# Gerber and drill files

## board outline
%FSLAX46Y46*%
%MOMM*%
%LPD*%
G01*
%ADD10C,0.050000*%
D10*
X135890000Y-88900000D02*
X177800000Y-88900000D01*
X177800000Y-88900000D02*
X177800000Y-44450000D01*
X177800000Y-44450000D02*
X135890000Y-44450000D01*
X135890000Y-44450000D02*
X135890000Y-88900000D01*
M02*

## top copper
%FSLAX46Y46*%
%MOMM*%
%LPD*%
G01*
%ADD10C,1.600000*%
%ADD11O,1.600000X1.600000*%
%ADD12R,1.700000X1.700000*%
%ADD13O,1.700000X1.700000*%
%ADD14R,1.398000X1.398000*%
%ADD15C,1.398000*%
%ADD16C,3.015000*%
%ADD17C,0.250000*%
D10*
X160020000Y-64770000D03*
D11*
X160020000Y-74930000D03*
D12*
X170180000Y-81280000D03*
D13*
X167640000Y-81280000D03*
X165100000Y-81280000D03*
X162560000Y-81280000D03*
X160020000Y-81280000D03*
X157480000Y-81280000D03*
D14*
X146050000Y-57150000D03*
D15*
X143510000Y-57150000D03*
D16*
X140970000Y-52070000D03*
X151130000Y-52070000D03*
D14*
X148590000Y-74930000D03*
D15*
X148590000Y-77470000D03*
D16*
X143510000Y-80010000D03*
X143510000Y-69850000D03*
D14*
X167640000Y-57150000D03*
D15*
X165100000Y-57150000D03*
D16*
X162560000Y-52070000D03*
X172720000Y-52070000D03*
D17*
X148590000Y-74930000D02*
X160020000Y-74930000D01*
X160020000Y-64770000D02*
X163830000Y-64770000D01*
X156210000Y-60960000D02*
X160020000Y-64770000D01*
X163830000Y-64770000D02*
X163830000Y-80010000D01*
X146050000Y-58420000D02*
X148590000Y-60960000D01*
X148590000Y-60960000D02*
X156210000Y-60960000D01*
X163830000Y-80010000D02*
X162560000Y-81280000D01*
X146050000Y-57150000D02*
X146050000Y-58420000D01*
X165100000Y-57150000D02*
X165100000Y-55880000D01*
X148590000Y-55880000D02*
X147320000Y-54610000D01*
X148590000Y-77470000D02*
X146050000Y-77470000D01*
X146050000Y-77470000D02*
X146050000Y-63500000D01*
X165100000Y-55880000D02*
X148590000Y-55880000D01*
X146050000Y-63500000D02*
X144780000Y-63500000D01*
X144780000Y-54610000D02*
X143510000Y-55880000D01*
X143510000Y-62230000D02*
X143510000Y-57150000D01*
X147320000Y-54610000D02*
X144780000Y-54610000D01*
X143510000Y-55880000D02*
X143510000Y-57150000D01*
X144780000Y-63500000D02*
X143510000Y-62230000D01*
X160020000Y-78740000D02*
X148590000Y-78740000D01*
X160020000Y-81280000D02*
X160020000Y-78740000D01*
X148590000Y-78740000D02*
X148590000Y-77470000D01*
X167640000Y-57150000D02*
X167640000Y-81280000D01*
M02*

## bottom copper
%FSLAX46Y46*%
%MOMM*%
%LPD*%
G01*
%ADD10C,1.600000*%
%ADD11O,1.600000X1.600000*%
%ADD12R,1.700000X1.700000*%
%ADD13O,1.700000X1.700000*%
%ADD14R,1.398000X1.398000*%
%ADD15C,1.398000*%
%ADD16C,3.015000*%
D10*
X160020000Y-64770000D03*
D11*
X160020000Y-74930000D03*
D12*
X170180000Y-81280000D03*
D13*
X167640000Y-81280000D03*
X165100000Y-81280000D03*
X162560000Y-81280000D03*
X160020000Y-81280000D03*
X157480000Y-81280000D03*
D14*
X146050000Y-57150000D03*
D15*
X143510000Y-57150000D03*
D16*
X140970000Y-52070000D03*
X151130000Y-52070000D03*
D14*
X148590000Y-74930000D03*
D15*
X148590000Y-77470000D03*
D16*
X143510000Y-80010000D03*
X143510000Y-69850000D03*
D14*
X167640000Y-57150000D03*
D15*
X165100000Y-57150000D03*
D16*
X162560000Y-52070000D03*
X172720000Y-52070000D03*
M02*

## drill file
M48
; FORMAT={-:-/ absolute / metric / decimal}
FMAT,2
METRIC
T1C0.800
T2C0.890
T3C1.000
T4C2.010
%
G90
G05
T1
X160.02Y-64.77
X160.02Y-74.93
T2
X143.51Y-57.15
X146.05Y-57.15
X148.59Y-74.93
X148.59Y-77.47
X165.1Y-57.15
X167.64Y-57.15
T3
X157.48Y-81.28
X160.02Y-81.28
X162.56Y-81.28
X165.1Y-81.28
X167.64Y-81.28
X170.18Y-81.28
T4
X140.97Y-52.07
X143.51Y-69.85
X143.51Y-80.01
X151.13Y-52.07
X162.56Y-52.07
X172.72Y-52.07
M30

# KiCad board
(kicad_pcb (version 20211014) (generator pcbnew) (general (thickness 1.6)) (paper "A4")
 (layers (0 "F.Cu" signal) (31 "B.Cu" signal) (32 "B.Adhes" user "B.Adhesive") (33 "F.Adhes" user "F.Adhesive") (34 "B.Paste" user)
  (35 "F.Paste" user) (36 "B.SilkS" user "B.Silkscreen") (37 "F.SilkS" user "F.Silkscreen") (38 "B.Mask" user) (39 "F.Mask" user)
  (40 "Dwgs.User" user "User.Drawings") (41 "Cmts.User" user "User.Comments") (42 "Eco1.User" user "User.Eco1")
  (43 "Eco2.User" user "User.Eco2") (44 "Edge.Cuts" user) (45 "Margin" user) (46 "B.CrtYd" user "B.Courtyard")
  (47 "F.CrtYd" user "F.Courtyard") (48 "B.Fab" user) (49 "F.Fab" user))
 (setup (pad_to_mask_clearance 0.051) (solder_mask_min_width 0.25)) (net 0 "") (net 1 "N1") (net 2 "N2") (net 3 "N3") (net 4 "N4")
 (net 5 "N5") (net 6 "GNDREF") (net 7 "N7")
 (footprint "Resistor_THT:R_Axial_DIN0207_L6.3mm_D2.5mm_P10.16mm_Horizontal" (layer "F.Cu") (at 160.02 64.77 -90)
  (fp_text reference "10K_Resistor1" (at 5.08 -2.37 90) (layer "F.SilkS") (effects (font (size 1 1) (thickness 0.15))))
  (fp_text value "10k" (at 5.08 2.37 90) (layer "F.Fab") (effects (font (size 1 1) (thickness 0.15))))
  (pad "1" thru_hole circle locked (at 0 0 270) (size 1.6 1.6) (drill 0.8) (layers *.Cu *.Mask) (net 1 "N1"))
  (pad "2" thru_hole oval locked (at 10.16 0 270) (size 1.6 1.6) (drill 0.8) (layers *.Cu *.Mask) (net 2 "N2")))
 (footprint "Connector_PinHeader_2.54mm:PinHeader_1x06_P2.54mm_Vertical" (layer "F.Cu") (at 170.18 81.28 -90)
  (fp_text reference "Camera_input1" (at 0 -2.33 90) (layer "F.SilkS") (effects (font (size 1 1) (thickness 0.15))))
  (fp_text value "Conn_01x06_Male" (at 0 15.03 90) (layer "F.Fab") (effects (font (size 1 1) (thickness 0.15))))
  (pad "1" thru_hole rect locked (at 0 0 270) (size 1.7 1.7) (drill 1) (layers *.Cu *.Mask) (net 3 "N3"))
  (pad "2" thru_hole oval locked (at 0 2.54 270) (size 1.7 1.7) (drill 1) (layers *.Cu *.Mask) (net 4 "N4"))
  (pad "3" thru_hole oval locked (at 0 5.08 270) (size 1.7 1.7) (drill 1) (layers *.Cu *.Mask) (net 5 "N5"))
  (pad "4" thru_hole oval locked (at 0 7.62 270) (size 1.7 1.7) (drill 1) (layers *.Cu *.Mask) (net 1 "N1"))
  (pad "5" thru_hole oval locked (at 0 10.16 270) (size 1.7 1.7) (drill 1) (layers *.Cu *.Mask) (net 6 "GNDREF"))
  (pad "6" thru_hole oval locked (at 0 12.7 270) (size 1.7 1.7) (drill 1) (layers *.Cu *.Mask) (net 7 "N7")))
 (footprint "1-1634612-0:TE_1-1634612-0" (layer "F.Cu") (at 146.05 57.15 90)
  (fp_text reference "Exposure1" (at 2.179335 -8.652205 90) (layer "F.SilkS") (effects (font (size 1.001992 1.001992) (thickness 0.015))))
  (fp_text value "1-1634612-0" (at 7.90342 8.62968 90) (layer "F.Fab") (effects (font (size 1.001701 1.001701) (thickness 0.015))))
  (pad "1" thru_hole rect locked (at 0 0 90) (size 1.398 1.398) (drill 0.89) (layers *.Cu *.Mask) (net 1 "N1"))
  (pad "2" thru_hole circle locked (at 0 -2.54 90) (size 1.398 1.398) (drill 0.89) (layers *.Cu *.Mask) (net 6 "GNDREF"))
  (pad "S1" thru_hole circle locked (at 5.08 -5.08 90) (size 3.015 3.015) (drill 2.01) (layers *.Cu *.Mask))
  (pad "S2" thru_hole circle locked (at 5.08 5.08 90) (size 3.015 3.015) (drill 2.01) (layers *.Cu *.Mask)))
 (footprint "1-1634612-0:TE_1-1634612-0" (layer "F.Cu") (at 148.59 74.93 180)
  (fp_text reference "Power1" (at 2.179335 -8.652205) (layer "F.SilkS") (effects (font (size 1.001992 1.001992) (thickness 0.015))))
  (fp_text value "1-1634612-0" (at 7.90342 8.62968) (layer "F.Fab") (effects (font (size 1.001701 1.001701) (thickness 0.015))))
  (pad "1" thru_hole rect locked (at 0 0 180) (size 1.398 1.398) (drill 0.89) (layers *.Cu *.Mask) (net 2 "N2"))
  (pad "2" thru_hole circle locked (at 0 -2.54 180) (size 1.398 1.398) (drill 0.89) (layers *.Cu *.Mask) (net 6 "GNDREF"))
  (pad "S1" thru_hole circle locked (at 5.08 -5.08 180) (size 3.015 3.015) (drill 2.01) (layers *.Cu *.Mask))
  (pad "S2" thru_hole circle locked (at 5.08 5.08 180) (size 3.015 3.015) (drill 2.01) (layers *.Cu *.Mask)))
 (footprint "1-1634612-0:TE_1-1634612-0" (layer "F.Cu") (at 167.64 57.15 90)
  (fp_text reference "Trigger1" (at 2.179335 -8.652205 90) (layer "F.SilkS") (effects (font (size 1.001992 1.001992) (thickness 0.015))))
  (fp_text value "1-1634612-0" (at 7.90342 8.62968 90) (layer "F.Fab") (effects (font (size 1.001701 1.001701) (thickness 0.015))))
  (pad "1" thru_hole rect locked (at 0 0 90) (size 1.398 1.398) (drill 0.89) (layers *.Cu *.Mask) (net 4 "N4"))
  (pad "2" thru_hole circle locked (at 0 -2.54 90) (size 1.398 1.398) (drill 0.89) (layers *.Cu *.Mask) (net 6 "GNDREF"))
  (pad "S1" thru_hole circle locked (at 5.08 -5.08 90) (size 3.015 3.015) (drill 2.01) (layers *.Cu *.Mask))
  (pad "S2" thru_hole circle locked (at 5.08 5.08 90) (size 3.015 3.015) (drill 2.01) (layers *.Cu *.Mask)))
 (gr_line (start 135.89 88.9) (end 177.8 88.9) (layer "Edge.Cuts") (width 0.05))
 (gr_line (start 177.8 88.9) (end 177.8 44.45) (layer "Edge.Cuts") (width 0.05))
 (gr_line (start 177.8 44.45) (end 135.89 44.45) (layer "Edge.Cuts") (width 0.05))
 (gr_line (start 135.89 44.45) (end 135.89 88.9) (layer "Edge.Cuts") (width 0.05))
 (segment (start 148.59 74.93) (end 160.02 74.93) (width 0.25) (layer "F.Cu") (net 2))
 (segment (start 160.02 64.77) (end 163.83 64.77) (width 0.25) (layer "F.Cu") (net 1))
 (segment (start 156.21 60.96) (end 160.02 64.77) (width 0.25) (layer "F.Cu") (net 1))
 (segment (start 163.83 64.77) (end 163.83 80.01) (width 0.25) (layer "F.Cu") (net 1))
 (segment (start 146.05 58.42) (end 148.59 60.96) (width 0.25) (layer "F.Cu") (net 1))
 (segment (start 148.59 60.96) (end 156.21 60.96) (width 0.25) (layer "F.Cu") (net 1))
 (segment (start 163.83 80.01) (end 162.56 81.28) (width 0.25) (layer "F.Cu") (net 1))
 (segment (start 146.05 57.15) (end 146.05 58.42) (width 0.25) (layer "F.Cu") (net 1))
 (segment (start 165.1 57.15) (end 165.1 55.88) (width 0.25) (layer "F.Cu") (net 6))
 (segment (start 148.59 55.88) (end 147.32 54.61) (width 0.25) (layer "F.Cu") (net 6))
 (segment (start 148.59 77.47) (end 146.05 77.47) (width 0.25) (layer "F.Cu") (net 6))
 (segment (start 146.05 77.47) (end 146.05 63.5) (width 0.25) (layer "F.Cu") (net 6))
 (segment (start 165.1 55.88) (end 148.59 55.88) (width 0.25) (layer "F.Cu") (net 6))
 (segment (start 146.05 63.5) (end 144.78 63.5) (width 0.25) (layer "F.Cu") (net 6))
 (segment (start 144.78 54.61) (end 143.51 55.88) (width 0.25) (layer "F.Cu") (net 6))
 (segment (start 143.51 62.23) (end 143.51 57.15) (width 0.25) (layer "F.Cu") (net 6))
 (segment (start 147.32 54.61) (end 144.78 54.61) (width 0.25) (layer "F.Cu") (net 6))
 (segment (start 143.51 55.88) (end 143.51 57.15) (width 0.25) (layer "F.Cu") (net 6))
 (segment (start 144.78 63.5) (end 143.51 62.23) (width 0.25) (layer "F.Cu") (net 6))
 (segment (start 160.02 78.74) (end 148.59 78.74) (width 0.25) (layer "F.Cu") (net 6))
 (segment (start 160.02 81.28) (end 160.02 78.74) (width 0.25) (layer "F.Cu") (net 6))
 (segment (start 148.59 78.74) (end 148.59 77.47) (width 0.25) (layer "F.Cu") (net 6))
 (segment (start 167.64 57.15) (end 167.64 81.28) (width 0.25) (layer "F.Cu") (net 4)))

